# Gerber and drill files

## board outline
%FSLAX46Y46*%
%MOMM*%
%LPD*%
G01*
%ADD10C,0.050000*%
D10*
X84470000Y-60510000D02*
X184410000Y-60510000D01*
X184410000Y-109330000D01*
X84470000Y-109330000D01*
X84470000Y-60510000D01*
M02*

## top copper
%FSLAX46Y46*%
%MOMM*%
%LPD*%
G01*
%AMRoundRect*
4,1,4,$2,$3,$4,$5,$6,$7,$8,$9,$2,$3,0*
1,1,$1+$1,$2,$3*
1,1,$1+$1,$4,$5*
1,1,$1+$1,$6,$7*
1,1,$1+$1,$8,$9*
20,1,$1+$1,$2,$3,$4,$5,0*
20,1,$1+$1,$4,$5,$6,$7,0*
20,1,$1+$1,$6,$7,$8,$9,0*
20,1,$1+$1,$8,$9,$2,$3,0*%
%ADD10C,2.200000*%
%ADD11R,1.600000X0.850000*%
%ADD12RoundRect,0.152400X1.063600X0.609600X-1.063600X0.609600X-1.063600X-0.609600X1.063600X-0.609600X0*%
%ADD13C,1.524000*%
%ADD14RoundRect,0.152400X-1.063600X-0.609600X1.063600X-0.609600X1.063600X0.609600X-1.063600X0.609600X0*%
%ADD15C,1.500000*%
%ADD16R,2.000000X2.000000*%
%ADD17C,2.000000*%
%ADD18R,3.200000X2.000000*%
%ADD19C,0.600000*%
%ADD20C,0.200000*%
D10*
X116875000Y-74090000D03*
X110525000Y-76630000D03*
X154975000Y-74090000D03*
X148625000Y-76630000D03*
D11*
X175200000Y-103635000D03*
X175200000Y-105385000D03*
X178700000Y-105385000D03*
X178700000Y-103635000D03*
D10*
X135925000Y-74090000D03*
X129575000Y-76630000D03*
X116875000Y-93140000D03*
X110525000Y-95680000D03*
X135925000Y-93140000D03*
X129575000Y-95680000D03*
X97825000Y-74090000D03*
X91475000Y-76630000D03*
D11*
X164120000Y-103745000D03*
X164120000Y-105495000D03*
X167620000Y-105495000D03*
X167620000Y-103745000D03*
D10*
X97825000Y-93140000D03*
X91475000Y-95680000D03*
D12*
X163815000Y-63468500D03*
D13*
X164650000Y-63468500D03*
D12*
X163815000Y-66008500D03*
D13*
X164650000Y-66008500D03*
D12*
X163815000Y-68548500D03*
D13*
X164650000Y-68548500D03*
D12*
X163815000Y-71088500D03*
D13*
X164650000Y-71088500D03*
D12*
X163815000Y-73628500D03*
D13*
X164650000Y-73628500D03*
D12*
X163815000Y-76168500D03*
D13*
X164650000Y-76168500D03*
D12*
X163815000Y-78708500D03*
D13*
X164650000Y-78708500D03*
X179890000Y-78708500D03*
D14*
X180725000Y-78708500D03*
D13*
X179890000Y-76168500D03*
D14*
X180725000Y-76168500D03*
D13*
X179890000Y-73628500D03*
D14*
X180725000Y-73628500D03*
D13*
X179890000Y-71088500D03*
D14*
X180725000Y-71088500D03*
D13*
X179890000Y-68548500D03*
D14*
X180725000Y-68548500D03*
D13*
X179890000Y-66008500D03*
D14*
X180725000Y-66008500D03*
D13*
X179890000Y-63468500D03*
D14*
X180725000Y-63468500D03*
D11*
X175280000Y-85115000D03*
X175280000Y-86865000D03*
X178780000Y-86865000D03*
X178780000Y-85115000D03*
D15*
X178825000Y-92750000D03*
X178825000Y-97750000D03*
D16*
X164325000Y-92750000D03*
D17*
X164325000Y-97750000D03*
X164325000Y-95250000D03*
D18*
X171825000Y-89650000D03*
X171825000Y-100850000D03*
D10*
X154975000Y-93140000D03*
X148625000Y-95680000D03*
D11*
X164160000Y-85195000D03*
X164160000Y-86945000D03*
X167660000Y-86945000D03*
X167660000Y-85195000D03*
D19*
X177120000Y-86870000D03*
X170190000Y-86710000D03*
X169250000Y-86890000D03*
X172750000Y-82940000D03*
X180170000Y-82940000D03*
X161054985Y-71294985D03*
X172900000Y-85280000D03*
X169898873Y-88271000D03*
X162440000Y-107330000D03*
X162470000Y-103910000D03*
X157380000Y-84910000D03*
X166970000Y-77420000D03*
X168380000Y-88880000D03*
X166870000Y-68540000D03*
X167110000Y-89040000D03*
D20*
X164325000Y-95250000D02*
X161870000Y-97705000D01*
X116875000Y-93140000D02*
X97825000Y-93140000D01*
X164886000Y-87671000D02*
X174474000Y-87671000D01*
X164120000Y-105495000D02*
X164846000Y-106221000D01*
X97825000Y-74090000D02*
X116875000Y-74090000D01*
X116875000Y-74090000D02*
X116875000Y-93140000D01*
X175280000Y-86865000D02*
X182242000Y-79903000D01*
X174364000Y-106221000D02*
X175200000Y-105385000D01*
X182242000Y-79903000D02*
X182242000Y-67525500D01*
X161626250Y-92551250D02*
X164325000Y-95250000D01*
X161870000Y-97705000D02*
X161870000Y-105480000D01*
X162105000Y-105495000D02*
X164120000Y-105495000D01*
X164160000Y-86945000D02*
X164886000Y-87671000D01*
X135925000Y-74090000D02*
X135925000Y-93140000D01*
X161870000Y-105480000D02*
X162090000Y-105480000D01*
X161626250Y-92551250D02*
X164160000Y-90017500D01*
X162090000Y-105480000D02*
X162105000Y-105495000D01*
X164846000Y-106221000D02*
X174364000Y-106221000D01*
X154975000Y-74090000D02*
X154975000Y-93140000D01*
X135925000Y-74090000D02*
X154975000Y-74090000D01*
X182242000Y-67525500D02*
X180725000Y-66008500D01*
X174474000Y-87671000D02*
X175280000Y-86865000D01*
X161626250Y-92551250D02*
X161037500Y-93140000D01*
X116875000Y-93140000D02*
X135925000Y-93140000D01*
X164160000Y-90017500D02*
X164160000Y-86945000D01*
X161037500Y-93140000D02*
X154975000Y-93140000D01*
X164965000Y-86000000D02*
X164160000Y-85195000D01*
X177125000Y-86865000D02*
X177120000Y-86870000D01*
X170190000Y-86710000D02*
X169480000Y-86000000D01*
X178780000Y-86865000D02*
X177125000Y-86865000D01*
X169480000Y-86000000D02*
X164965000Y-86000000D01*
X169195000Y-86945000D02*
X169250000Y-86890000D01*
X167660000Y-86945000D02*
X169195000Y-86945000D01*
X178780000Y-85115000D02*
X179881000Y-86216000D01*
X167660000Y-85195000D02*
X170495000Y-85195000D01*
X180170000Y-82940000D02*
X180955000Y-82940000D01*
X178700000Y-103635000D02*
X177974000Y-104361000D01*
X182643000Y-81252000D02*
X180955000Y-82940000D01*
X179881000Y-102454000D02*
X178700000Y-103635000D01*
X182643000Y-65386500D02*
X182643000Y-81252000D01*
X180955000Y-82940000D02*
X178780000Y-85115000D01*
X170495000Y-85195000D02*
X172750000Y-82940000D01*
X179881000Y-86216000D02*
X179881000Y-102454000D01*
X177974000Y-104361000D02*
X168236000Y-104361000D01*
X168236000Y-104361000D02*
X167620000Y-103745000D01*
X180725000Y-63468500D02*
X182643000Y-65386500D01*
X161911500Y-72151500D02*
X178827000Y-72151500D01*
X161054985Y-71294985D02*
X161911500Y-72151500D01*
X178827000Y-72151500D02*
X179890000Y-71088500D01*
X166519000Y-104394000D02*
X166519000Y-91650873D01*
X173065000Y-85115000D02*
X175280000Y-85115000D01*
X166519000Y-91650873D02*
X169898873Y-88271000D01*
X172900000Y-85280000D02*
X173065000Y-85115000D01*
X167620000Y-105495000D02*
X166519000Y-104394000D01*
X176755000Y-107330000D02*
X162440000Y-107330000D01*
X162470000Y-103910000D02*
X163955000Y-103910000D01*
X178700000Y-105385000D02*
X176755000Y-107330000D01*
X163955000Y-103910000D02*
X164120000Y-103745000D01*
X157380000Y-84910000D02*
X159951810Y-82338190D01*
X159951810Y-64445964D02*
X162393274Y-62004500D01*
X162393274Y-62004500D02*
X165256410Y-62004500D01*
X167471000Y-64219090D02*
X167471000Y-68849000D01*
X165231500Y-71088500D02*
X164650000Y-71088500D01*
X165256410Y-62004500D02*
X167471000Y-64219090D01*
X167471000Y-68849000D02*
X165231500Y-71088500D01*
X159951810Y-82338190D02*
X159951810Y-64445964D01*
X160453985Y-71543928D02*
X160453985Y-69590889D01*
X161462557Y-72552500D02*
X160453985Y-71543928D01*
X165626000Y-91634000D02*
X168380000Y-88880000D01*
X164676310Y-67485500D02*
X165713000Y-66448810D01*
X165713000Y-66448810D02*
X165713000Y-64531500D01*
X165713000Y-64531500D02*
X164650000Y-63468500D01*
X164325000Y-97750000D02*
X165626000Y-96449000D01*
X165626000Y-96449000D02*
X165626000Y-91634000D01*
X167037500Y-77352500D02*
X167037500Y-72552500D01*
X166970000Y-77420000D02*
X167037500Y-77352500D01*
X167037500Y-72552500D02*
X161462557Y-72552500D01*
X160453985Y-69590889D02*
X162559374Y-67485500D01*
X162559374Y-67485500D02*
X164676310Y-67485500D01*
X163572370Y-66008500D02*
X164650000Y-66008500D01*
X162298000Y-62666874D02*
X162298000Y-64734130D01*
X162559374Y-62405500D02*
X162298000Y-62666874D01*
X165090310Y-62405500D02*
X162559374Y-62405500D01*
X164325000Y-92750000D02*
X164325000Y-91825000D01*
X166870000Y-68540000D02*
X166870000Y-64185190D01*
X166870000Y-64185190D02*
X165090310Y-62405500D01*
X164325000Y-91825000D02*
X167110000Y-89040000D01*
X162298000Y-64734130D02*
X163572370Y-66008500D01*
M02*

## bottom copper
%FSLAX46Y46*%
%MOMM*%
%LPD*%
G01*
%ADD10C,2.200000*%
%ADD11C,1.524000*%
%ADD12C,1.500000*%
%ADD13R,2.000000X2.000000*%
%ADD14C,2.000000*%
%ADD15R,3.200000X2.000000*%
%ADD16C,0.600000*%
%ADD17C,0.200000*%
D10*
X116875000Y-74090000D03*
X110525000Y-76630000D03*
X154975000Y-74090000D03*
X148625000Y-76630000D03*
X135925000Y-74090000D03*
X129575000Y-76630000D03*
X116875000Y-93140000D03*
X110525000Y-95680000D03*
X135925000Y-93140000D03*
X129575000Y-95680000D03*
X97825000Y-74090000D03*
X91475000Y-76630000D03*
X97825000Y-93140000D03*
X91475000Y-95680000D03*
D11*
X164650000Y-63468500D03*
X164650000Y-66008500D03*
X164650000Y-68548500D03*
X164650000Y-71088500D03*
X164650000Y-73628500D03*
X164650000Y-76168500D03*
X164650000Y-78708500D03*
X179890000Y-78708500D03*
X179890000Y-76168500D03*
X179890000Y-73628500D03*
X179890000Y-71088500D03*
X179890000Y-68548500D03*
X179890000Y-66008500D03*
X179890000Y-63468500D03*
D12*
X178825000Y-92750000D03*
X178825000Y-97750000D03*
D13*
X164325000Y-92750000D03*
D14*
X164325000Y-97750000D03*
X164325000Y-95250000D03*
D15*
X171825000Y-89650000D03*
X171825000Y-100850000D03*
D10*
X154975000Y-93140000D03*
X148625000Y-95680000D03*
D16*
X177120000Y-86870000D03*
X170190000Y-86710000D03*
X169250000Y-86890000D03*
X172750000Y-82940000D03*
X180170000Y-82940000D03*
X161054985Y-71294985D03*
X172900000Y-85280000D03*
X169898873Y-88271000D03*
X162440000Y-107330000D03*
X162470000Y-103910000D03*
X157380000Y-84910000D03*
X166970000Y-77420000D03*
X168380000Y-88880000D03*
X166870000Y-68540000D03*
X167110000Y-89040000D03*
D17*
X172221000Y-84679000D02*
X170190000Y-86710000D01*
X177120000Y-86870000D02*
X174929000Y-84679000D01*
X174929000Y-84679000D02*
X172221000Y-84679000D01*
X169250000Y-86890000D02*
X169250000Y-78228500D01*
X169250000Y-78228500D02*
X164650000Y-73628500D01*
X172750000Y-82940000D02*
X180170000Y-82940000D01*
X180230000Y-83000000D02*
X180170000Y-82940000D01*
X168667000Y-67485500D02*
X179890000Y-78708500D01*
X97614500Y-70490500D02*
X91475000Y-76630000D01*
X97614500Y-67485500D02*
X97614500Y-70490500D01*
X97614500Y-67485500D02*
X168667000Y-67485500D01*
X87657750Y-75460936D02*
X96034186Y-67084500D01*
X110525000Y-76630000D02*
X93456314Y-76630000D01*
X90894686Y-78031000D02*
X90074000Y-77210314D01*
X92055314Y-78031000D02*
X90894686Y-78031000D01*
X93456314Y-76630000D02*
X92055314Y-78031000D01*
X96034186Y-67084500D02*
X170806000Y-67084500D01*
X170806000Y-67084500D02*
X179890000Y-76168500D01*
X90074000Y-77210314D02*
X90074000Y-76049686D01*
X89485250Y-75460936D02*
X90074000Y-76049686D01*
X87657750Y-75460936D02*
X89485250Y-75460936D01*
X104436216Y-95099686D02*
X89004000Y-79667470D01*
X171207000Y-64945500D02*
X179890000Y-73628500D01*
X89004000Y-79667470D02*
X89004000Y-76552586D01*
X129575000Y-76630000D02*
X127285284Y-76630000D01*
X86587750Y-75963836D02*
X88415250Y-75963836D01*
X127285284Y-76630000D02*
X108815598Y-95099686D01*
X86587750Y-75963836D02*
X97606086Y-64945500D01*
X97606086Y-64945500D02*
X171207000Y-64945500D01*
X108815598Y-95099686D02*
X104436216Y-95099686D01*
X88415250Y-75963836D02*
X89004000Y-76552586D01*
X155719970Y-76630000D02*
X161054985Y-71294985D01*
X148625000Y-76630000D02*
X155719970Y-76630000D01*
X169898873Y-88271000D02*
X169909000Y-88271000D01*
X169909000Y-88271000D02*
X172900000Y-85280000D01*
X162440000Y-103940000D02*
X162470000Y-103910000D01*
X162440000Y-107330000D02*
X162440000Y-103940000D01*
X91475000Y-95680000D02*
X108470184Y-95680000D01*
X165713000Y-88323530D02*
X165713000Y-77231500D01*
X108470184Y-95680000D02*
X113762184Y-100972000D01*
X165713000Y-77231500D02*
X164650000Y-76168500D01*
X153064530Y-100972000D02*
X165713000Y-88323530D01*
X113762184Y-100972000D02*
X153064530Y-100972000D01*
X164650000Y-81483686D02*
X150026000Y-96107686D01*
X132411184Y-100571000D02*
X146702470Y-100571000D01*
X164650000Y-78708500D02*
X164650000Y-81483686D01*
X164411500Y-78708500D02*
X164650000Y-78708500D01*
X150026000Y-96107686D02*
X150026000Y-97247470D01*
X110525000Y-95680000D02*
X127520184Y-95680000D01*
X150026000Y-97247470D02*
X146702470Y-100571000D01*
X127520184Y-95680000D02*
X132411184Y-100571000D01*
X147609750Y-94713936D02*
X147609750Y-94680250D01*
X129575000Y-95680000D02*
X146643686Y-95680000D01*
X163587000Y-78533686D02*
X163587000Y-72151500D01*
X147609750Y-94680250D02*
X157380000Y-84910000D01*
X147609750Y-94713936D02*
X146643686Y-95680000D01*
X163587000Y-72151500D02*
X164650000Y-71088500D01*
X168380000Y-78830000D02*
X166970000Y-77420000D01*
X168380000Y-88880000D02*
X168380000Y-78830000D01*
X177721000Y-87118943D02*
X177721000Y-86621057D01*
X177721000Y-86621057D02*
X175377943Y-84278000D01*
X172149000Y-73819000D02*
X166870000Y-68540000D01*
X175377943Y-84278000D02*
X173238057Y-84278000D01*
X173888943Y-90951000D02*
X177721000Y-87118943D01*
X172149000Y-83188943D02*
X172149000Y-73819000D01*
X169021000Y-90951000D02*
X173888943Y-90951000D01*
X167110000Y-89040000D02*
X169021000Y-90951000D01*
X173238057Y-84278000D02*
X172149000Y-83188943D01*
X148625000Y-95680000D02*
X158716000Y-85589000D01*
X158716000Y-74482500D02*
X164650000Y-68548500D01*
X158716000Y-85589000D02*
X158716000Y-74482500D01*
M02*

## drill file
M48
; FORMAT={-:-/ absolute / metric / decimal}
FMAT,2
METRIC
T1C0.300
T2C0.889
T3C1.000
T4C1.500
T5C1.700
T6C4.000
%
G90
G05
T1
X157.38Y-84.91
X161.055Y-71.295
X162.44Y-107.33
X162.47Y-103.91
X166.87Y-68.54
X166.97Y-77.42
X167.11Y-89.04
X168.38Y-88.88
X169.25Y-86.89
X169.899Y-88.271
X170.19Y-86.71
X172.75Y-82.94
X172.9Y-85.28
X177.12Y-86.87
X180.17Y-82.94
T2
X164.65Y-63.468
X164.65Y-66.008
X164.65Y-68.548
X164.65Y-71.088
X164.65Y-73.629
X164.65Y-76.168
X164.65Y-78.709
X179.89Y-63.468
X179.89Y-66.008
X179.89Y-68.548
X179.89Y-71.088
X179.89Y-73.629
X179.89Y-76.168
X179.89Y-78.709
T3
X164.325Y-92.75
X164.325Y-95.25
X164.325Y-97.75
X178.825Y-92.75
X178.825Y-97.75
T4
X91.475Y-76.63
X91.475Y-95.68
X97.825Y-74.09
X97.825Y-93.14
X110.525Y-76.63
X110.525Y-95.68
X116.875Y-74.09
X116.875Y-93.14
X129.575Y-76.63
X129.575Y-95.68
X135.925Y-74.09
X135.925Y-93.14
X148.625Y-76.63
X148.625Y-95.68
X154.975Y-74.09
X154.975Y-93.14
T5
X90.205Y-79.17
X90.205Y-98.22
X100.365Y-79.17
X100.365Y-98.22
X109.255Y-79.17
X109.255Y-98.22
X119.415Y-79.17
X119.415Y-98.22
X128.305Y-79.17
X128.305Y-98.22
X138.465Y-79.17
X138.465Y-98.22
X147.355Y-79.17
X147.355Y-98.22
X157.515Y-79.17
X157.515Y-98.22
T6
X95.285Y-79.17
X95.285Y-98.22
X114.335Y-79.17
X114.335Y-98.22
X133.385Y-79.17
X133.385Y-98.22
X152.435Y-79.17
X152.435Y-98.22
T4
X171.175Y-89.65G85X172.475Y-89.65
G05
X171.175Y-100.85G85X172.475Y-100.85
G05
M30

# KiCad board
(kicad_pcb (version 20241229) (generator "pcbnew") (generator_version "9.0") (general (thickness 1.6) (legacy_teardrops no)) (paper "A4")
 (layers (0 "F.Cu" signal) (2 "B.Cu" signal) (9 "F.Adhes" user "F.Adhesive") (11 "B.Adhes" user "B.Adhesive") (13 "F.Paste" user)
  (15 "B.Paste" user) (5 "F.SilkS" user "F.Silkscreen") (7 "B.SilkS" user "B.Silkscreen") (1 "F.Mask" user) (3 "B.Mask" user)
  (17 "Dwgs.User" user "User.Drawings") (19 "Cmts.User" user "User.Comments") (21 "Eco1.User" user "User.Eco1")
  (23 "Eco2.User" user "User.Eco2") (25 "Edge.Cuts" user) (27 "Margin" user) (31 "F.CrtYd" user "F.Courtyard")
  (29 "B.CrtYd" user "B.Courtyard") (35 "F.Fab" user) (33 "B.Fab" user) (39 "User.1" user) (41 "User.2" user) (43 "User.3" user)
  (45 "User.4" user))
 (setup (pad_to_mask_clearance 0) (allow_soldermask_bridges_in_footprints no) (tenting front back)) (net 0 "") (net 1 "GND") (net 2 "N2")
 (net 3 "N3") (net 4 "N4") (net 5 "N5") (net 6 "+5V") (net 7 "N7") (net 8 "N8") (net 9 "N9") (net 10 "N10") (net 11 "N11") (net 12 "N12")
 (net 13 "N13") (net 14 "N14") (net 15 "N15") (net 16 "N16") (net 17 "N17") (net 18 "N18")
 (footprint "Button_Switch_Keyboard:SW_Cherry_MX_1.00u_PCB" (layer "F.Cu") (at 116.875 74.09)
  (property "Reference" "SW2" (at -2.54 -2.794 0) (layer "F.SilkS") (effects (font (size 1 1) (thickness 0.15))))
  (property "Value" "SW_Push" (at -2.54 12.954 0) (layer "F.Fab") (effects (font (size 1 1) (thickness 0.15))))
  (pad "" np_thru_hole circle (at -7.62 5.08) (size 1.7 1.7) (drill 1.7) (layers "*.Cu" "*.Mask"))
  (pad "" np_thru_hole circle (at -2.54 5.08) (size 4 4) (drill 4) (layers "*.Cu" "*.Mask"))
  (pad "" np_thru_hole circle (at 2.54 5.08) (size 1.7 1.7) (drill 1.7) (layers "*.Cu" "*.Mask"))
  (pad "1" thru_hole circle (at 0 0) (size 2.2 2.2) (drill 1.5) (layers "*.Cu" "*.Mask") (remove_unused_layers no) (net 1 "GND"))
  (pad "2" thru_hole circle (at -6.35 2.54) (size 2.2 2.2) (drill 1.5) (layers "*.Cu" "*.Mask") (remove_unused_layers no) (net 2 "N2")))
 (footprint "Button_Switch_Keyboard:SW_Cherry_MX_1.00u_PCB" (layer "F.Cu") (at 154.975 74.09)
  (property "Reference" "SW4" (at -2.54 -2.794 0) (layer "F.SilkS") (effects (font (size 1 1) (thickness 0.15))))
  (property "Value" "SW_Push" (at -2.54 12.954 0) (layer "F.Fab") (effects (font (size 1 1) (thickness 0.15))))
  (pad "" np_thru_hole circle (at -7.62 5.08) (size 1.7 1.7) (drill 1.7) (layers "*.Cu" "*.Mask"))
  (pad "" np_thru_hole circle (at -2.54 5.08) (size 4 4) (drill 4) (layers "*.Cu" "*.Mask"))
  (pad "" np_thru_hole circle (at 2.54 5.08) (size 1.7 1.7) (drill 1.7) (layers "*.Cu" "*.Mask"))
  (pad "1" thru_hole circle (at 0 0) (size 2.2 2.2) (drill 1.5) (layers "*.Cu" "*.Mask") (remove_unused_layers no) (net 1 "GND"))
  (pad "2" thru_hole circle (at -6.35 2.54) (size 2.2 2.2) (drill 1.5) (layers "*.Cu" "*.Mask") (remove_unused_layers no) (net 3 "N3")))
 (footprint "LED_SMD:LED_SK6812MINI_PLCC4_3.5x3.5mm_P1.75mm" (layer "F.Cu") (at 176.95 104.51)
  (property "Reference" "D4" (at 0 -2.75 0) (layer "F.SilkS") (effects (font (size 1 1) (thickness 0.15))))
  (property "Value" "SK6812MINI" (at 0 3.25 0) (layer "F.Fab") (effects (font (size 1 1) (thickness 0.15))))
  (pad "1" smd rect (at -1.75 -0.875) (size 1.6 0.85) (layers "F.Cu" "F.Mask" "F.Paste") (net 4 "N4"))
  (pad "2" smd rect (at -1.75 0.875) (size 1.6 0.85) (layers "F.Cu" "F.Mask" "F.Paste") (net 1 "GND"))
  (pad "3" smd rect (at 1.75 0.875) (size 1.6 0.85) (layers "F.Cu" "F.Mask" "F.Paste") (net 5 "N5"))
  (pad "4" smd rect (at 1.75 -0.875) (size 1.6 0.85) (layers "F.Cu" "F.Mask" "F.Paste") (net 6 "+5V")))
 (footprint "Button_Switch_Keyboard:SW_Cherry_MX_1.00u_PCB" (layer "F.Cu") (at 135.925 74.09)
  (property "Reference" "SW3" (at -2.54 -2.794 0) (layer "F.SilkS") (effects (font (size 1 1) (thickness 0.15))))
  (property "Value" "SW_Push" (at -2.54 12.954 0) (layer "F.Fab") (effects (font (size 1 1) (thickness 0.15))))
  (pad "" np_thru_hole circle (at -7.62 5.08) (size 1.7 1.7) (drill 1.7) (layers "*.Cu" "*.Mask"))
  (pad "" np_thru_hole circle (at -2.54 5.08) (size 4 4) (drill 4) (layers "*.Cu" "*.Mask"))
  (pad "" np_thru_hole circle (at 2.54 5.08) (size 1.7 1.7) (drill 1.7) (layers "*.Cu" "*.Mask"))
  (pad "1" thru_hole circle (at 0 0) (size 2.2 2.2) (drill 1.5) (layers "*.Cu" "*.Mask") (remove_unused_layers no) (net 1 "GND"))
  (pad "2" thru_hole circle (at -6.35 2.54) (size 2.2 2.2) (drill 1.5) (layers "*.Cu" "*.Mask") (remove_unused_layers no) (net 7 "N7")))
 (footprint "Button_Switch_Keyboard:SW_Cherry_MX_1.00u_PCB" (layer "F.Cu") (at 116.875 93.14)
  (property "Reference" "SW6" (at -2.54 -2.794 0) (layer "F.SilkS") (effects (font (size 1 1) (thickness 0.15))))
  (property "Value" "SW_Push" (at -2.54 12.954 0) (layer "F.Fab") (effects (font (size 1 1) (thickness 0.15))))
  (pad "" np_thru_hole circle (at -7.62 5.08) (size 1.7 1.7) (drill 1.7) (layers "*.Cu" "*.Mask"))
  (pad "" np_thru_hole circle (at -2.54 5.08) (size 4 4) (drill 4) (layers "*.Cu" "*.Mask"))
  (pad "" np_thru_hole circle (at 2.54 5.08) (size 1.7 1.7) (drill 1.7) (layers "*.Cu" "*.Mask"))
  (pad "1" thru_hole circle (at 0 0) (size 2.2 2.2) (drill 1.5) (layers "*.Cu" "*.Mask") (remove_unused_layers no) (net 1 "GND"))
  (pad "2" thru_hole circle (at -6.35 2.54) (size 2.2 2.2) (drill 1.5) (layers "*.Cu" "*.Mask") (remove_unused_layers no) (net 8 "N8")))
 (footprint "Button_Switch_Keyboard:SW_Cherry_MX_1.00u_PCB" (layer "F.Cu") (at 135.925 93.14)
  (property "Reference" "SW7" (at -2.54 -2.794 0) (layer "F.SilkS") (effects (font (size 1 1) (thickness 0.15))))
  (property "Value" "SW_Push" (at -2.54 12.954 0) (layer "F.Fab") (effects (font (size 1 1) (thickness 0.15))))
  (pad "" np_thru_hole circle (at -7.62 5.08) (size 1.7 1.7) (drill 1.7) (layers "*.Cu" "*.Mask"))
  (pad "" np_thru_hole circle (at -2.54 5.08) (size 4 4) (drill 4) (layers "*.Cu" "*.Mask"))
  (pad "" np_thru_hole circle (at 2.54 5.08) (size 1.7 1.7) (drill 1.7) (layers "*.Cu" "*.Mask"))
  (pad "1" thru_hole circle (at 0 0) (size 2.2 2.2) (drill 1.5) (layers "*.Cu" "*.Mask") (remove_unused_layers no) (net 1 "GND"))
  (pad "2" thru_hole circle (at -6.35 2.54) (size 2.2 2.2) (drill 1.5) (layers "*.Cu" "*.Mask") (remove_unused_layers no) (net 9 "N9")))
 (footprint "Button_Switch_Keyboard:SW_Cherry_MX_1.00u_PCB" (layer "F.Cu") (at 97.825 74.09)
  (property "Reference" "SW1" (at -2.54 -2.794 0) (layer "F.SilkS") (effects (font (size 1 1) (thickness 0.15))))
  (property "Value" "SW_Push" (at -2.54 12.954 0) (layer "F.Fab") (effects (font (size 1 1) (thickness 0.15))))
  (pad "" np_thru_hole circle (at -7.62 5.08) (size 1.7 1.7) (drill 1.7) (layers "*.Cu" "*.Mask"))
  (pad "" np_thru_hole circle (at -2.54 5.08) (size 4 4) (drill 4) (layers "*.Cu" "*.Mask"))
  (pad "" np_thru_hole circle (at 2.54 5.08) (size 1.7 1.7) (drill 1.7) (layers "*.Cu" "*.Mask"))
  (pad "1" thru_hole circle (at 0 0) (size 2.2 2.2) (drill 1.5) (layers "*.Cu" "*.Mask") (remove_unused_layers no) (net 1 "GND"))
  (pad "2" thru_hole circle (at -6.35 2.54) (size 2.2 2.2) (drill 1.5) (layers "*.Cu" "*.Mask") (remove_unused_layers no) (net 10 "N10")))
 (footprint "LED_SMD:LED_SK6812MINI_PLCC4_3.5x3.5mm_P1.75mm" (layer "F.Cu") (at 165.87 104.62)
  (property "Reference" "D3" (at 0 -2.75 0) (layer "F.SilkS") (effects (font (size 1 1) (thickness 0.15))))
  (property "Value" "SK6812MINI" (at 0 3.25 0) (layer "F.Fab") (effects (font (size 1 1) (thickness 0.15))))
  (pad "1" smd rect (at -1.75 -0.875) (size 1.6 0.85) (layers "F.Cu" "F.Mask" "F.Paste") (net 5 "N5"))
  (pad "2" smd rect (at -1.75 0.875) (size 1.6 0.85) (layers "F.Cu" "F.Mask" "F.Paste") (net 1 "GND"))
  (pad "3" smd rect (at 1.75 0.875) (size 1.6 0.85) (layers "F.Cu" "F.Mask" "F.Paste") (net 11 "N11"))
  (pad "4" smd rect (at 1.75 -0.875) (size 1.6 0.85) (layers "F.Cu" "F.Mask" "F.Paste") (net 6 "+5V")))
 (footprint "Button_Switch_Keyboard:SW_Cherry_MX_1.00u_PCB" (layer "F.Cu") (at 97.825 93.14)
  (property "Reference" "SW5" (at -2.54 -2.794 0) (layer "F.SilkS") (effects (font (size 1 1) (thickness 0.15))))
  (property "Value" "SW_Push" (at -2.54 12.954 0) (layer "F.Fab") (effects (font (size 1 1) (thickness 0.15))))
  (pad "" np_thru_hole circle (at -7.62 5.08) (size 1.7 1.7) (drill 1.7) (layers "*.Cu" "*.Mask"))
  (pad "" np_thru_hole circle (at -2.54 5.08) (size 4 4) (drill 4) (layers "*.Cu" "*.Mask"))
  (pad "" np_thru_hole circle (at 2.54 5.08) (size 1.7 1.7) (drill 1.7) (layers "*.Cu" "*.Mask"))
  (pad "1" thru_hole circle (at 0 0) (size 2.2 2.2) (drill 1.5) (layers "*.Cu" "*.Mask") (remove_unused_layers no) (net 1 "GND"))
  (pad "2" thru_hole circle (at -6.35 2.54) (size 2.2 2.2) (drill 1.5) (layers "*.Cu" "*.Mask") (remove_unused_layers no) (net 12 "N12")))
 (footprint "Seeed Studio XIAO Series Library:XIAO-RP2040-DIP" (layer "F.Cu") (at 172.27 71.0885)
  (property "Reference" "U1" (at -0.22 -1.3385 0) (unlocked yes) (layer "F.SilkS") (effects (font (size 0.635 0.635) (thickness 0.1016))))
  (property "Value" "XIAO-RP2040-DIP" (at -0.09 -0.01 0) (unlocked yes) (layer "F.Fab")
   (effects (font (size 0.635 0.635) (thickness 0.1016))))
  (pad "1" smd roundrect (at -8.455 -7.62 180) (size 2.432 1.524) (layers "F.Cu" "F.Mask") (roundrect_rratio 0.1) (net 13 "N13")
   (thermal_bridge_angle 45))
  (pad "1" thru_hole circle (at -7.62 -7.62 180) (size 1.524 1.524) (drill 0.889) (layers "*.Cu" "*.Mask") (remove_unused_layers no)
   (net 13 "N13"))
  (pad "2" smd roundrect (at -8.455 -5.08 180) (size 2.432 1.524) (layers "F.Cu" "F.Mask") (roundrect_rratio 0.1) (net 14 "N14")
   (thermal_bridge_angle 45))
  (pad "2" thru_hole circle (at -7.62 -5.08 180) (size 1.524 1.524) (drill 0.889) (layers "*.Cu" "*.Mask") (remove_unused_layers no)
   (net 14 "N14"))
  (pad "3" smd roundrect (at -8.455 -2.54 180) (size 2.432 1.524) (layers "F.Cu" "F.Mask") (roundrect_rratio 0.1) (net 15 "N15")
   (thermal_bridge_angle 45))
  (pad "3" thru_hole circle (at -7.62 -2.54 180) (size 1.524 1.524) (drill 0.889) (layers "*.Cu" "*.Mask") (remove_unused_layers no)
   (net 15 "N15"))
  (pad "4" smd roundrect (at -8.455 0 180) (size 2.432 1.524) (layers "F.Cu" "F.Mask") (roundrect_rratio 0.1) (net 9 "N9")
   (thermal_bridge_angle 45))
  (pad "4" thru_hole circle (at -7.62 0 180) (size 1.524 1.524) (drill 0.889) (layers "*.Cu" "*.Mask") (remove_unused_layers no)
   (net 9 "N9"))
  (pad "5" smd roundrect (at -8.455 2.54 180) (size 2.432 1.524) (layers "F.Cu" "F.Mask") (roundrect_rratio 0.1) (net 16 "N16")
   (thermal_bridge_angle 45))
  (pad "5" thru_hole circle (at -7.62 2.54 180) (size 1.524 1.524) (drill 0.889) (layers "*.Cu" "*.Mask") (remove_unused_layers no)
   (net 16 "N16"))
  (pad "6" smd roundrect (at -8.455 5.08 180) (size 2.432 1.524) (layers "F.Cu" "F.Mask") (roundrect_rratio 0.1) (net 12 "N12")
   (thermal_bridge_angle 45))
  (pad "6" thru_hole circle (at -7.62 5.08 180) (size 1.524 1.524) (drill 0.889) (layers "*.Cu" "*.Mask") (remove_unused_layers no)
   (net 12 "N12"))
  (pad "7" smd roundrect (at -8.455 7.62 180) (size 2.432 1.524) (layers "F.Cu" "F.Mask") (roundrect_rratio 0.1) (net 8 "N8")
   (thermal_bridge_angle 45))
  (pad "7" thru_hole circle (at -7.62 7.62 180) (size 1.524 1.524) (drill 0.889) (layers "*.Cu" "*.Mask") (remove_unused_layers no)
   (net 8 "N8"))
  (pad "8" thru_hole circle (at 7.62 7.62) (size 1.524 1.524) (drill 0.889) (layers "*.Cu" "*.Mask") (remove_unused_layers no)
   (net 10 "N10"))
  (pad "8" smd roundrect (at 8.455 7.62) (size 2.432 1.524) (layers "F.Cu" "F.Mask") (roundrect_rratio 0.1) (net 10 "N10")
   (thermal_bridge_angle 45))
  (pad "9" thru_hole circle (at 7.62 5.08) (size 1.524 1.524) (drill 0.889) (layers "*.Cu" "*.Mask") (remove_unused_layers no) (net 2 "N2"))
  (pad "9" smd roundrect (at 8.455 5.08) (size 2.432 1.524) (layers "F.Cu" "F.Mask") (roundrect_rratio 0.1) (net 2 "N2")
   (thermal_bridge_angle 45))
  (pad "10" thru_hole circle (at 7.62 2.54) (size 1.524 1.524) (drill 0.889) (layers "*.Cu" "*.Mask") (remove_unused_layers no) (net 7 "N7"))
  (pad "10" smd roundrect (at 8.455 2.54) (size 2.432 1.524) (layers "F.Cu" "F.Mask") (roundrect_rratio 0.1) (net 7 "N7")
   (thermal_bridge_angle 45))
  (pad "11" thru_hole circle (at 7.62 0) (size 1.524 1.524) (drill 0.889) (layers "*.Cu" "*.Mask") (remove_unused_layers no) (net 3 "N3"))
  (pad "11" smd roundrect (at 8.455 0) (size 2.432 1.524) (layers "F.Cu" "F.Mask") (roundrect_rratio 0.1) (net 3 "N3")
   (thermal_bridge_angle 45))
  (pad "12" thru_hole circle (at 7.62 -2.54) (size 1.524 1.524) (drill 0.889) (layers "*.Cu" "*.Mask") (remove_unused_layers no)
   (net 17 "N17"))
  (pad "12" smd roundrect (at 8.455 -2.54) (size 2.432 1.524) (layers "F.Cu" "F.Mask") (roundrect_rratio 0.1) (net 17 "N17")
   (thermal_bridge_angle 45))
  (pad "13" thru_hole circle (at 7.62 -5.08) (size 1.524 1.524) (drill 0.889) (layers "*.Cu" "*.Mask") (remove_unused_layers no)
   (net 1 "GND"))
  (pad "13" smd roundrect (at 8.455 -5.08) (size 2.432 1.524) (layers "F.Cu" "F.Mask") (roundrect_rratio 0.1) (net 1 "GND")
   (thermal_bridge_angle 45))
  (pad "14" thru_hole circle (at 7.62 -7.62) (size 1.524 1.524) (drill 0.889) (layers "*.Cu" "*.Mask") (remove_unused_layers no)
   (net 6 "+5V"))
  (pad "14" smd roundrect (at 8.455 -7.62) (size 2.432 1.524) (layers "F.Cu" "F.Mask") (roundrect_rratio 0.1) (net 6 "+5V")
   (thermal_bridge_angle 45)))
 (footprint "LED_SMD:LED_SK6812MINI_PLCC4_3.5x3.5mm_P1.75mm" (layer "F.Cu") (at 177.03 85.99)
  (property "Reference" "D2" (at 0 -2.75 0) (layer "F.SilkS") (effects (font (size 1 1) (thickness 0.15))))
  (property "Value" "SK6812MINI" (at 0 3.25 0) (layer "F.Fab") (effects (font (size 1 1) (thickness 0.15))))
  (pad "1" smd rect (at -1.75 -0.875) (size 1.6 0.85) (layers "F.Cu" "F.Mask" "F.Paste") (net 11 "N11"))
  (pad "2" smd rect (at -1.75 0.875) (size 1.6 0.85) (layers "F.Cu" "F.Mask" "F.Paste") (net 1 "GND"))
  (pad "3" smd rect (at 1.75 0.875) (size 1.6 0.85) (layers "F.Cu" "F.Mask" "F.Paste") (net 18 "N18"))
  (pad "4" smd rect (at 1.75 -0.875) (size 1.6 0.85) (layers "F.Cu" "F.Mask" "F.Paste") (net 6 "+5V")))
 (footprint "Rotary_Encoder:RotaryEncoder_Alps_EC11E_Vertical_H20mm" (layer "F.Cu") (at 164.325 92.75)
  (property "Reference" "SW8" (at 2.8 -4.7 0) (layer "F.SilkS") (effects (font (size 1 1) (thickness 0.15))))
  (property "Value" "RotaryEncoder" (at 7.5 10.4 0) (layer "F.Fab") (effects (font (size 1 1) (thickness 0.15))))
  (pad "" thru_hole circle (at 14.5 0) (size 1.5 1.5) (drill 1) (layers "*.Cu" "*.Mask") (remove_unused_layers no))
  (pad "" thru_hole circle (at 14.5 5) (size 1.5 1.5) (drill 1) (layers "*.Cu" "*.Mask") (remove_unused_layers no))
  (pad "A" thru_hole rect (at 0 0) (size 2 2) (drill 1) (layers "*.Cu" "*.Mask") (remove_unused_layers no) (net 14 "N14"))
  (pad "B" thru_hole circle (at 0 5) (size 2 2) (drill 1) (layers "*.Cu" "*.Mask") (remove_unused_layers no) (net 13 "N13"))
  (pad "C" thru_hole circle (at 0 2.5) (size 2 2) (drill 1) (layers "*.Cu" "*.Mask") (remove_unused_layers no) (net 1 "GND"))
  (pad "MP" thru_hole rect (at 7.5 -3.1) (size 3.2 2) (drill oval 2.8 1.5) (layers "*.Cu" "*.Mask") (remove_unused_layers no))
  (pad "MP" thru_hole rect (at 7.5 8.1) (size 3.2 2) (drill oval 2.8 1.5) (layers "*.Cu" "*.Mask") (remove_unused_layers no)))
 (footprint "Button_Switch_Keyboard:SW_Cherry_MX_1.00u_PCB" (layer "F.Cu") (at 154.975 93.14)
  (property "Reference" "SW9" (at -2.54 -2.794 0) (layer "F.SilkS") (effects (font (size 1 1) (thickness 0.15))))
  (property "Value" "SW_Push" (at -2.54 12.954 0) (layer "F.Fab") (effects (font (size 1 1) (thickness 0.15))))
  (pad "" np_thru_hole circle (at -7.62 5.08) (size 1.7 1.7) (drill 1.7) (layers "*.Cu" "*.Mask"))
  (pad "" np_thru_hole circle (at -2.54 5.08) (size 4 4) (drill 4) (layers "*.Cu" "*.Mask"))
  (pad "" np_thru_hole circle (at 2.54 5.08) (size 1.7 1.7) (drill 1.7) (layers "*.Cu" "*.Mask"))
  (pad "1" thru_hole circle (at 0 0) (size 2.2 2.2) (drill 1.5) (layers "*.Cu" "*.Mask") (remove_unused_layers no) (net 1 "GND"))
  (pad "2" thru_hole circle (at -6.35 2.54) (size 2.2 2.2) (drill 1.5) (layers "*.Cu" "*.Mask") (remove_unused_layers no) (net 15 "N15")))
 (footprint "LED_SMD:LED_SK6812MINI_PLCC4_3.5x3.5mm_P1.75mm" (layer "F.Cu") (at 165.91 86.07)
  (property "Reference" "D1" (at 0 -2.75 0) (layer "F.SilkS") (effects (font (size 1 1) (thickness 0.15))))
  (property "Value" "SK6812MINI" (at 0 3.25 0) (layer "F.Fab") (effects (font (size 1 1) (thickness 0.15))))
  (pad "1" smd rect (at -1.75 -0.875) (size 1.6 0.85) (layers "F.Cu" "F.Mask" "F.Paste") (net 18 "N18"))
  (pad "2" smd rect (at -1.75 0.875) (size 1.6 0.85) (layers "F.Cu" "F.Mask" "F.Paste") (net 1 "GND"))
  (pad "3" smd rect (at 1.75 0.875) (size 1.6 0.85) (layers "F.Cu" "F.Mask" "F.Paste") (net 16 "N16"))
  (pad "4" smd rect (at 1.75 -0.875) (size 1.6 0.85) (layers "F.Cu" "F.Mask" "F.Paste") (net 6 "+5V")))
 (gr_rect (start 84.47 60.51) (end 184.41 109.33) (stroke (width 0.05) (type default)) (fill no) (layer "Edge.Cuts"))
 (segment (start 164.325 95.25) (end 161.87 97.705) (width 0.2) (layer "F.Cu") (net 1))
 (segment (start 116.875 93.14) (end 97.825 93.14) (width 0.2) (layer "F.Cu") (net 1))
 (segment (start 164.886 87.671) (end 174.474 87.671) (width 0.2) (layer "F.Cu") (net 1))
 (segment (start 164.12 105.495) (end 164.846 106.221) (width 0.2) (layer "F.Cu") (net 1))
 (segment (start 97.825 74.09) (end 116.875 74.09) (width 0.2) (layer "F.Cu") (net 1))
 (segment (start 116.875 74.09) (end 116.875 93.14) (width 0.2) (layer "F.Cu") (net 1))
 (segment (start 175.28 86.865) (end 182.242 79.903) (width 0.2) (layer "F.Cu") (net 1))
 (segment (start 174.364 106.221) (end 175.2 105.385) (width 0.2) (layer "F.Cu") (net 1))
 (segment (start 182.242 79.903) (end 182.242 67.5255) (width 0.2) (layer "F.Cu") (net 1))
 (segment (start 161.62625 92.55125) (end 164.325 95.25) (width 0.2) (layer "F.Cu") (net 1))
 (segment (start 161.87 97.705) (end 161.87 105.48) (width 0.2) (layer "F.Cu") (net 1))
 (segment (start 162.105 105.495) (end 164.12 105.495) (width 0.2) (layer "F.Cu") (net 1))
 (segment (start 164.16 86.945) (end 164.886 87.671) (width 0.2) (layer "F.Cu") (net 1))
 (segment (start 135.925 74.09) (end 135.925 93.14) (width 0.2) (layer "F.Cu") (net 1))
 (segment (start 161.87 105.48) (end 162.09 105.48) (width 0.2) (layer "F.Cu") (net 1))
 (segment (start 161.62625 92.55125) (end 164.16 90.0175) (width 0.2) (layer "F.Cu") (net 1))
 (segment (start 162.09 105.48) (end 162.105 105.495) (width 0.2) (layer "F.Cu") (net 1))
 (segment (start 164.846 106.221) (end 174.364 106.221) (width 0.2) (layer "F.Cu") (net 1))
 (segment (start 154.975 74.09) (end 154.975 93.14) (width 0.2) (layer "F.Cu") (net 1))
 (segment (start 135.925 74.09) (end 154.975 74.09) (width 0.2) (layer "F.Cu") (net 1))
 (segment (start 182.242 67.5255) (end 180.725 66.0085) (width 0.2) (layer "F.Cu") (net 1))
 (segment (start 174.474 87.671) (end 175.28 86.865) (width 0.2) (layer "F.Cu") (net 1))
 (segment (start 161.62625 92.55125) (end 161.0375 93.14) (width 0.2) (layer "F.Cu") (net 1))
 (segment (start 116.875 93.14) (end 135.925 93.14) (width 0.2) (layer "F.Cu") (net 1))
 (segment (start 164.16 90.0175) (end 164.16 86.945) (width 0.2) (layer "F.Cu") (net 1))
 (segment (start 161.0375 93.14) (end 154.975 93.14) (width 0.2) (layer "F.Cu") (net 1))
 (segment (start 164.965 86) (end 164.16 85.195) (width 0.2) (layer "F.Cu") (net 18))
 (segment (start 177.125 86.865) (end 177.12 86.87) (width 0.2) (layer "F.Cu") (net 18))
 (segment (start 170.19 86.71) (end 169.48 86) (width 0.2) (layer "F.Cu") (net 18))
 (segment (start 178.78 86.865) (end 177.125 86.865) (width 0.2) (layer "F.Cu") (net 18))
 (segment (start 169.48 86) (end 164.965 86) (width 0.2) (layer "F.Cu") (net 18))
 (via (at 177.12 86.87) (size 0.6) (drill 0.3) (layers "F.Cu" "B.Cu") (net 18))
 (via (at 170.19 86.71) (size 0.6) (drill 0.3) (layers "F.Cu" "B.Cu") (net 18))
 (segment (start 172.221 84.679) (end 170.19 86.71) (width 0.2) (layer "B.Cu") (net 18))
 (segment (start 177.12 86.87) (end 174.929 84.679) (width 0.2) (layer "B.Cu") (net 18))
 (segment (start 174.929 84.679) (end 172.221 84.679) (width 0.2) (layer "B.Cu") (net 18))
 (segment (start 169.195 86.945) (end 169.25 86.89) (width 0.2) (layer "F.Cu") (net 16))
 (segment (start 167.66 86.945) (end 169.195 86.945) (width 0.2) (layer "F.Cu") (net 16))
 (via (at 169.25 86.89) (size 0.6) (drill 0.3) (layers "F.Cu" "B.Cu") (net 16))
 (segment (start 169.25 86.89) (end 169.25 78.2285) (width 0.2) (layer "B.Cu") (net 16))
 (segment (start 169.25 78.2285) (end 164.65 73.6285) (width 0.2) (layer "B.Cu") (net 16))
 (segment (start 178.78 85.115) (end 179.881 86.216) (width 0.2) (layer "F.Cu") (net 6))
 (segment (start 167.66 85.195) (end 170.495 85.195) (width 0.2) (layer "F.Cu") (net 6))
 (segment (start 180.17 82.94) (end 180.955 82.94) (width 0.2) (layer "F.Cu") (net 6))
 (segment (start 178.7 103.635) (end 177.974 104.361) (width 0.2) (layer "F.Cu") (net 6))
 (segment (start 182.643 81.252) (end 180.955 82.94) (width 0.2) (layer "F.Cu") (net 6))
 (segment (start 179.881 102.454) (end 178.7 103.635) (width 0.2) (layer "F.Cu") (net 6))
 (segment (start 182.643 65.3865) (end 182.643 81.252) (width 0.2) (layer "F.Cu") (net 6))
 (segment (start 180.955 82.94) (end 178.78 85.115) (width 0.2) (layer "F.Cu") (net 6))
 (segment (start 170.495 85.195) (end 172.75 82.94) (width 0.2) (layer "F.Cu") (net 6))
 (segment (start 179.881 86.216) (end 179.881 102.454) (width 0.2) (layer "F.Cu") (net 6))
 (segment (start 177.974 104.361) (end 168.236 104.361) (width 0.2) (layer "F.Cu") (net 6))
 (segment (start 168.236 104.361) (end 167.62 103.745) (width 0.2) (layer "F.Cu") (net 6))
 (segment (start 180.725 63.4685) (end 182.643 65.3865) (width 0.2) (layer "F.Cu") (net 6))
 (via (at 172.75 82.94) (size 0.6) (drill 0.3) (layers "F.Cu" "B.Cu") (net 6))
 (via (at 180.17 82.94) (size 0.6) (drill 0.3) (layers "F.Cu" "B.Cu") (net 6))
 (segment (start 172.75 82.94) (end 180.17 82.94) (width 0.2) (layer "B.Cu") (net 6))
 (segment (start 180.23 83) (end 180.17 82.94) (width 0.2) (layer "B.Cu") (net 6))
 (segment (start 168.667 67.4855) (end 179.89 78.7085) (width 0.2) (layer "B.Cu") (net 10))
 (segment (start 97.6145 70.4905) (end 91.475 76.63) (width 0.2) (layer "B.Cu") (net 10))
 (segment (start 97.6145 67.4855) (end 97.6145 70.4905) (width 0.2) (layer "B.Cu") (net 10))
 (segment (start 97.6145 67.4855) (end 168.667 67.4855) (width 0.2) (layer "B.Cu") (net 10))
 (segment (start 87.65775 75.460936) (end 96.034186 67.0845) (width 0.2) (layer "B.Cu") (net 2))
 (segment (start 110.525 76.63) (end 93.456314 76.63) (width 0.2) (layer "B.Cu") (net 2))
 (segment (start 90.894686 78.031) (end 90.074 77.210314) (width 0.2) (layer "B.Cu") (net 2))
 (segment (start 92.055314 78.031) (end 90.894686 78.031) (width 0.2) (layer "B.Cu") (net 2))
 (segment (start 93.456314 76.63) (end 92.055314 78.031) (width 0.2) (layer "B.Cu") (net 2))
 (segment (start 96.034186 67.0845) (end 170.806 67.0845) (width 0.2) (layer "B.Cu") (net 2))
 (segment (start 170.806 67.0845) (end 179.89 76.1685) (width 0.2) (layer "B.Cu") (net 2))
 (segment (start 90.074 77.210314) (end 90.074 76.049686) (width 0.2) (layer "B.Cu") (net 2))
 (segment (start 89.48525 75.460936) (end 90.074 76.049686) (width 0.2) (layer "B.Cu") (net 2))
 (segment (start 87.65775 75.460936) (end 89.48525 75.460936) (width 0.2) (layer "B.Cu") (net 2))
 (segment (start 104.436216 95.099686) (end 89.004 79.66747) (width 0.2) (layer "B.Cu") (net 7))
 (segment (start 171.207 64.9455) (end 179.89 73.6285) (width 0.2) (layer "B.Cu") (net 7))
 (segment (start 89.004 79.66747) (end 89.004 76.552586) (width 0.2) (layer "B.Cu") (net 7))
 (segment (start 129.575 76.63) (end 127.285284 76.63) (width 0.2) (layer "B.Cu") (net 7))
 (segment (start 86.58775 75.963836) (end 88.41525 75.963836) (width 0.2) (layer "B.Cu") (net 7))
 (segment (start 127.285284 76.63) (end 108.815598 95.099686) (width 0.2) (layer "B.Cu") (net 7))
 (segment (start 86.58775 75.963836) (end 97.606086 64.9455) (width 0.2) (layer "B.Cu") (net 7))
 (segment (start 97.606086 64.9455) (end 171.207 64.9455) (width 0.2) (layer "B.Cu") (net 7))
 (segment (start 108.815598 95.099686) (end 104.436216 95.099686) (width 0.2) (layer "B.Cu") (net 7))
 (segment (start 88.41525 75.963836) (end 89.004 76.552586) (width 0.2) (layer "B.Cu") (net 7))
 (segment (start 161.9115 72.1515) (end 178.827 72.1515) (width 0.2) (layer "F.Cu") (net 3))
 (segment (start 161.054985 71.294985) (end 161.9115 72.1515) (width 0.2) (layer "F.Cu") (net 3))
 (segment (start 178.827 72.1515) (end 179.89 71.0885) (width 0.2) (layer "F.Cu") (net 3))
 (via (at 161.054985 71.294985) (size 0.6) (drill 0.3) (layers "F.Cu" "B.Cu") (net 3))
 (segment (start 155.71997 76.63) (end 161.054985 71.294985) (width 0.2) (layer "B.Cu") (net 3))
 (segment (start 148.625 76.63) (end 155.71997 76.63) (width 0.2) (layer "B.Cu") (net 3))
 (segment (start 166.519 104.394) (end 166.519 91.650873) (width 0.2) (layer "F.Cu") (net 11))
 (segment (start 173.065 85.115) (end 175.28 85.115) (width 0.2) (layer "F.Cu") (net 11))
 (segment (start 166.519 91.650873) (end 169.898873 88.271) (width 0.2) (layer "F.Cu") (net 11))
 (segment (start 172.9 85.28) (end 173.065 85.115) (width 0.2) (layer "F.Cu") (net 11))
 (segment (start 167.62 105.495) (end 166.519 104.394) (width 0.2) (layer "F.Cu") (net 11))
 (via (at 172.9 85.28) (size 0.6) (drill 0.3) (layers "F.Cu" "B.Cu") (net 11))
 (via (at 169.898873 88.271) (size 0.6) (drill 0.3) (layers "F.Cu" "B.Cu") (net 11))
 (segment (start 169.898873 88.271) (end 169.909 88.271) (width 0.2) (layer "B.Cu") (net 11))
 (segment (start 169.909 88.271) (end 172.9 85.28) (width 0.2) (layer "B.Cu") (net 11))
 (segment (start 176.755 107.33) (end 162.44 107.33) (width 0.2) (layer "F.Cu") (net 5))
 (segment (start 162.47 103.91) (end 163.955 103.91) (width 0.2) (layer "F.Cu") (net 5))
 (segment (start 178.7 105.385) (end 176.755 107.33) (width 0.2) (layer "F.Cu") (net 5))
 (segment (start 163.955 103.91) (end 164.12 103.745) (width 0.2) (layer "F.Cu") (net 5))
 (via (at 162.44 107.33) (size 0.6) (drill 0.3) (layers "F.Cu" "B.Cu") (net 5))
 (via (at 162.47 103.91) (size 0.6) (drill 0.3) (layers "F.Cu" "B.Cu") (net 5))
 (segment (start 162.44 103.94) (end 162.47 103.91) (width 0.2) (layer "B.Cu") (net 5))
 (segment (start 162.44 107.33) (end 162.44 103.94) (width 0.2) (layer "B.Cu") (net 5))
 (segment (start 91.475 95.68) (end 108.470184 95.68) (width 0.2) (layer "B.Cu") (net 12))
 (segment (start 165.713 88.32353) (end 165.713 77.2315) (width 0.2) (layer "B.Cu") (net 12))
 (segment (start 108.470184 95.68) (end 113.762184 100.972) (width 0.2) (layer "B.Cu") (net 12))
 (segment (start 165.713 77.2315) (end 164.65 76.1685) (width 0.2) (layer "B.Cu") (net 12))
 (segment (start 153.06453 100.972) (end 165.713 88.32353) (width 0.2) (layer "B.Cu") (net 12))
 (segment (start 113.762184 100.972) (end 153.06453 100.972) (width 0.2) (layer "B.Cu") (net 12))
 (segment (start 164.65 81.483686) (end 150.026 96.107686) (width 0.2) (layer "B.Cu") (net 8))
 (segment (start 132.411184 100.571) (end 146.70247 100.571) (width 0.2) (layer "B.Cu") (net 8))
 (segment (start 164.65 78.7085) (end 164.65 81.483686) (width 0.2) (layer "B.Cu") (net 8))
 (segment (start 164.4115 78.7085) (end 164.65 78.7085) (width 0.2) (layer "B.Cu") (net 8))
 (segment (start 150.026 96.107686) (end 150.026 97.24747) (width 0.2) (layer "B.Cu") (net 8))
 (segment (start 110.525 95.68) (end 127.520184 95.68) (width 0.2) (layer "B.Cu") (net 8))
 (segment (start 150.026 97.24747) (end 146.70247 100.571) (width 0.2) (layer "B.Cu") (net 8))
 (segment (start 127.520184 95.68) (end 132.411184 100.571) (width 0.2) (layer "B.Cu") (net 8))
 (segment (start 157.38 84.91) (end 159.95181 82.33819) (width 0.2) (layer "F.Cu") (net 9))
 (segment (start 159.95181 64.445964) (end 162.393274 62.0045) (width 0.2) (layer "F.Cu") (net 9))
 (segment (start 162.393274 62.0045) (end 165.25641 62.0045) (width 0.2) (layer "F.Cu") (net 9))
 (segment (start 167.471 64.21909) (end 167.471 68.849) (width 0.2) (layer "F.Cu") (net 9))
 (segment (start 165.2315 71.0885) (end 164.65 71.0885) (width 0.2) (layer "F.Cu") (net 9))
 (segment (start 165.25641 62.0045) (end 167.471 64.21909) (width 0.2) (layer "F.Cu") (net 9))
 (segment (start 167.471 68.849) (end 165.2315 71.0885) (width 0.2) (layer "F.Cu") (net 9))
 (segment (start 159.95181 82.33819) (end 159.95181 64.445964) (width 0.2) (layer "F.Cu") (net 9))
 (via (at 157.38 84.91) (size 0.6) (drill 0.3) (layers "F.Cu" "B.Cu") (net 9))
 (segment (start 147.60975 94.713936) (end 147.60975 94.68025) (width 0.2) (layer "B.Cu") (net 9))
 (segment (start 129.575 95.68) (end 146.643686 95.68) (width 0.2) (layer "B.Cu") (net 9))
 (segment (start 163.587 78.533686) (end 163.587 72.1515) (width 0.2) (layer "B.Cu") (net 9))
 (segment (start 147.60975 94.68025) (end 157.38 84.91) (width 0.2) (layer "B.Cu") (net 9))
 (segment (start 147.60975 94.713936) (end 146.643686 95.68) (width 0.2) (layer "B.Cu") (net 9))
 (segment (start 163.587 72.1515) (end 164.65 71.0885) (width 0.2) (layer "B.Cu") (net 9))
 (segment (start 160.453985 71.543928) (end 160.453985 69.590889) (width 0.2) (layer "F.Cu") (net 13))
 (segment (start 161.462557 72.5525) (end 160.453985 71.543928) (width 0.2) (layer "F.Cu") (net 13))
 (segment (start 165.626 91.634) (end 168.38 88.88) (width 0.2) (layer "F.Cu") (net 13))
 (segment (start 164.67631 67.4855) (end 165.713 66.44881) (width 0.2) (layer "F.Cu") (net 13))
 (segment (start 165.713 66.44881) (end 165.713 64.5315) (width 0.2) (layer "F.Cu") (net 13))
 (segment (start 165.713 64.5315) (end 164.65 63.4685) (width 0.2) (layer "F.Cu") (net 13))
 (segment (start 164.325 97.75) (end 165.626 96.449) (width 0.2) (layer "F.Cu") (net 13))
 (segment (start 165.626 96.449) (end 165.626 91.634) (width 0.2) (layer "F.Cu") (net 13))
 (segment (start 167.0375 77.3525) (end 167.0375 72.5525) (width 0.2) (layer "F.Cu") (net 13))
 (segment (start 166.97 77.42) (end 167.0375 77.3525) (width 0.2) (layer "F.Cu") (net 13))
 (segment (start 167.0375 72.5525) (end 161.462557 72.5525) (width 0.2) (layer "F.Cu") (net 13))
 (segment (start 160.453985 69.590889) (end 162.559374 67.4855) (width 0.2) (layer "F.Cu") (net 13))
 (segment (start 162.559374 67.4855) (end 164.67631 67.4855) (width 0.2) (layer "F.Cu") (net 13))
 (via (at 166.97 77.42) (size 0.6) (drill 0.3) (layers "F.Cu" "B.Cu") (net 13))
 (via (at 168.38 88.88) (size 0.6) (drill 0.3) (layers "F.Cu" "B.Cu") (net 13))
 (segment (start 168.38 78.83) (end 166.97 77.42) (width 0.2) (layer "B.Cu") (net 13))
 (segment (start 168.38 88.88) (end 168.38 78.83) (width 0.2) (layer "B.Cu") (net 13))
 (segment (start 163.57237 66.0085) (end 164.65 66.0085) (width 0.2) (layer "F.Cu") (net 14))
 (segment (start 162.298 62.666874) (end 162.298 64.73413) (width 0.2) (layer "F.Cu") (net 14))
 (segment (start 162.559374 62.4055) (end 162.298 62.666874) (width 0.2) (layer "F.Cu") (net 14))
 (segment (start 165.09031 62.4055) (end 162.559374 62.4055) (width 0.2) (layer "F.Cu") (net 14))
 (segment (start 164.325 92.75) (end 164.325 91.825) (width 0.2) (layer "F.Cu") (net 14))
 (segment (start 166.87 68.54) (end 166.87 64.18519) (width 0.2) (layer "F.Cu") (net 14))
 (segment (start 166.87 64.18519) (end 165.09031 62.4055) (width 0.2) (layer "F.Cu") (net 14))
 (segment (start 164.325 91.825) (end 167.11 89.04) (width 0.2) (layer "F.Cu") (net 14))
 (segment (start 162.298 64.73413) (end 163.57237 66.0085) (width 0.2) (layer "F.Cu") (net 14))
 (via (at 166.87 68.54) (size 0.6) (drill 0.3) (layers "F.Cu" "B.Cu") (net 14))
 (via (at 167.11 89.04) (size 0.6) (drill 0.3) (layers "F.Cu" "B.Cu") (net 14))
 (segment (start 177.721 87.118943) (end 177.721 86.621057) (width 0.2) (layer "B.Cu") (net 14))
 (segment (start 177.721 86.621057) (end 175.377943 84.278) (width 0.2) (layer "B.Cu") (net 14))
 (segment (start 172.149 73.819) (end 166.87 68.54) (width 0.2) (layer "B.Cu") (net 14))
 (segment (start 175.377943 84.278) (end 173.238057 84.278) (width 0.2) (layer "B.Cu") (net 14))
 (segment (start 173.888943 90.951) (end 177.721 87.118943) (width 0.2) (layer "B.Cu") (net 14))
 (segment (start 172.149 83.188943) (end 172.149 73.819) (width 0.2) (layer "B.Cu") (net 14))
 (segment (start 169.021 90.951) (end 173.888943 90.951) (width 0.2) (layer "B.Cu") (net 14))
 (segment (start 167.11 89.04) (end 169.021 90.951) (width 0.2) (layer "B.Cu") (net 14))
 (segment (start 173.238057 84.278) (end 172.149 83.188943) (width 0.2) (layer "B.Cu") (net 14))
 (segment (start 148.625 95.68) (end 158.716 85.589) (width 0.2) (layer "B.Cu") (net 15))
 (segment (start 158.716 74.4825) (end 164.65 68.5485) (width 0.2) (layer "B.Cu") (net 15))
 (segment (start 158.716 85.589) (end 158.716 74.4825) (width 0.2) (layer "B.Cu") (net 15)))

